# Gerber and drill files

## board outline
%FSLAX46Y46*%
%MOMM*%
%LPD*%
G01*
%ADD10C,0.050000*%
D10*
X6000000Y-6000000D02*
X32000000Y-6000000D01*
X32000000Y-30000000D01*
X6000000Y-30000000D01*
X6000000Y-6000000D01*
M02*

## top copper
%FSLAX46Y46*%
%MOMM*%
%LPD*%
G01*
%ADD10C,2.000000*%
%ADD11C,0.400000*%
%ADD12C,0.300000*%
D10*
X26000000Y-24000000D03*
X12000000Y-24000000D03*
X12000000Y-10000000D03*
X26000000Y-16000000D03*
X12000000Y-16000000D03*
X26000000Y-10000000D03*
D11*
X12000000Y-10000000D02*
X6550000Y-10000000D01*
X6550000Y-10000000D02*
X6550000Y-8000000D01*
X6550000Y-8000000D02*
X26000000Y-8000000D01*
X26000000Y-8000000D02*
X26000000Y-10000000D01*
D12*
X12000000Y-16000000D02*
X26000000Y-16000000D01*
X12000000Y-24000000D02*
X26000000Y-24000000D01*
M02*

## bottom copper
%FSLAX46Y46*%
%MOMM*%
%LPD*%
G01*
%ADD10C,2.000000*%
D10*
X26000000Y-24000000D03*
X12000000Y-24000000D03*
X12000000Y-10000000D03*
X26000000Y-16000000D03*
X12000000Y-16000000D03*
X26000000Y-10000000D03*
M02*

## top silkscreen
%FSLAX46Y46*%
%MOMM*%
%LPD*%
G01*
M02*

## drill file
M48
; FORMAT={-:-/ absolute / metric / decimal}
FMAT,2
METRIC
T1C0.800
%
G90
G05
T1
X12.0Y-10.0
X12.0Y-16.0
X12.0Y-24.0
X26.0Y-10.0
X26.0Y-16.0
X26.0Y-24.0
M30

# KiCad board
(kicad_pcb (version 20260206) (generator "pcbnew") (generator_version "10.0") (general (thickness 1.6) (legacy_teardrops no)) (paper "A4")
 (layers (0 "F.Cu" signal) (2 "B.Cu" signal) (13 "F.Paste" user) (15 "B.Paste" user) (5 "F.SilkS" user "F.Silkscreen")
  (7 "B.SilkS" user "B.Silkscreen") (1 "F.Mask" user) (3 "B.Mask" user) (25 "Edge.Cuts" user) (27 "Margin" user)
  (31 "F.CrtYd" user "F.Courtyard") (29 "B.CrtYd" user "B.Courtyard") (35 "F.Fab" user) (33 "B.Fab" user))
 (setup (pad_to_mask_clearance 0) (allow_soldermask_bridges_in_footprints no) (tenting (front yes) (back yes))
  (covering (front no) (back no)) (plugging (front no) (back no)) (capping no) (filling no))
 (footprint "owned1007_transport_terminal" (layer "F.Cu") (at 26 24)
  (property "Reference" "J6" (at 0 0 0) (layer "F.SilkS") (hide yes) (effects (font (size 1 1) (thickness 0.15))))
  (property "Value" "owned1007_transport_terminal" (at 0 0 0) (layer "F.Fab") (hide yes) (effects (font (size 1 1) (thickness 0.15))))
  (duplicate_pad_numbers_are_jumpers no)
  (pad "1" thru_hole circle (at 0 0) (size 2 2) (drill 0.8) (layers "*.Cu" "*.Mask") (remove_unused_layers no) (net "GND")))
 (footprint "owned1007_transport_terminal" (layer "F.Cu") (at 12 24)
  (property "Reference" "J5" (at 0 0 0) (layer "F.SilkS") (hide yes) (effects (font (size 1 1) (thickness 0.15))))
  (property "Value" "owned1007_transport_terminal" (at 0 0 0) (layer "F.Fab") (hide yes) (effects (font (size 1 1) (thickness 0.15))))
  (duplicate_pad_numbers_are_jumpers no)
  (pad "1" thru_hole circle (at 0 0) (size 2 2) (drill 0.8) (layers "*.Cu" "*.Mask") (remove_unused_layers no) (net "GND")))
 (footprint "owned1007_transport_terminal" (layer "F.Cu") (at 12 10)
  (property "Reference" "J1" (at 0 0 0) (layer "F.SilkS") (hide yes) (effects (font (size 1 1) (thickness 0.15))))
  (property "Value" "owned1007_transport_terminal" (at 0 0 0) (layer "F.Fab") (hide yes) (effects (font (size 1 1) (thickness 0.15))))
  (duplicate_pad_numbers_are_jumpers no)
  (pad "1" thru_hole circle (at 0 0) (size 2 2) (drill 0.8) (layers "*.Cu" "*.Mask") (remove_unused_layers no) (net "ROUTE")))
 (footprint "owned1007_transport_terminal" (layer "F.Cu") (at 26 16)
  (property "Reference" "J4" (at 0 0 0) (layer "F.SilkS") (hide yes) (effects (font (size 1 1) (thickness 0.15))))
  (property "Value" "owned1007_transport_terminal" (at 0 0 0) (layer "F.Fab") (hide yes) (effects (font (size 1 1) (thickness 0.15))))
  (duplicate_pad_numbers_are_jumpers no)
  (pad "1" thru_hole circle (at 0 0) (size 2 2) (drill 0.8) (layers "*.Cu" "*.Mask") (remove_unused_layers no) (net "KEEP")))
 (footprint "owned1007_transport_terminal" (layer "F.Cu") (at 12 16)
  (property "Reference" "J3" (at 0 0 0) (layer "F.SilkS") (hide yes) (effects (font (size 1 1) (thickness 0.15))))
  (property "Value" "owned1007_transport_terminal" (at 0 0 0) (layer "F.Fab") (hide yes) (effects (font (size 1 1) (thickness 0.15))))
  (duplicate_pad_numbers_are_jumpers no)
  (pad "1" thru_hole circle (at 0 0) (size 2 2) (drill 0.8) (layers "*.Cu" "*.Mask") (remove_unused_layers no) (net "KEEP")))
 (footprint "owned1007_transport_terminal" (layer "F.Cu") (at 26 10)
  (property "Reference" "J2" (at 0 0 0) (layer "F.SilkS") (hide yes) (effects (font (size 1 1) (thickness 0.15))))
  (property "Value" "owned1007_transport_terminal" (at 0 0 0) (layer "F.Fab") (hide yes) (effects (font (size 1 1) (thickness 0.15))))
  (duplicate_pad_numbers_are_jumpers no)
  (pad "1" thru_hole circle (at 0 0) (size 2 2) (drill 0.8) (layers "*.Cu" "*.Mask") (remove_unused_layers no) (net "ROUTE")))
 (gr_rect (start 6 6) (end 32 30) (stroke (width 0.05) (type default)) (fill no) (layer "Edge.Cuts"))
 (segment (start 12 10) (end 6.55 10) (width 0.4) (layer "F.Cu") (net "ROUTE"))
 (segment (start 6.55 10) (end 6.55 8) (width 0.4) (layer "F.Cu") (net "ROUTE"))
 (segment (start 6.55 8) (end 26 8) (width 0.4) (layer "F.Cu") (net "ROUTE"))
 (segment (start 26 8) (end 26 10) (width 0.4) (layer "F.Cu") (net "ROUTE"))
 (segment (start 12 16) (end 26 16) (width 0.3) (locked yes) (layer "F.Cu") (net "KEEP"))
 (segment (start 12 24) (end 26 24) (width 0.3) (layer "F.Cu") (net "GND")))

